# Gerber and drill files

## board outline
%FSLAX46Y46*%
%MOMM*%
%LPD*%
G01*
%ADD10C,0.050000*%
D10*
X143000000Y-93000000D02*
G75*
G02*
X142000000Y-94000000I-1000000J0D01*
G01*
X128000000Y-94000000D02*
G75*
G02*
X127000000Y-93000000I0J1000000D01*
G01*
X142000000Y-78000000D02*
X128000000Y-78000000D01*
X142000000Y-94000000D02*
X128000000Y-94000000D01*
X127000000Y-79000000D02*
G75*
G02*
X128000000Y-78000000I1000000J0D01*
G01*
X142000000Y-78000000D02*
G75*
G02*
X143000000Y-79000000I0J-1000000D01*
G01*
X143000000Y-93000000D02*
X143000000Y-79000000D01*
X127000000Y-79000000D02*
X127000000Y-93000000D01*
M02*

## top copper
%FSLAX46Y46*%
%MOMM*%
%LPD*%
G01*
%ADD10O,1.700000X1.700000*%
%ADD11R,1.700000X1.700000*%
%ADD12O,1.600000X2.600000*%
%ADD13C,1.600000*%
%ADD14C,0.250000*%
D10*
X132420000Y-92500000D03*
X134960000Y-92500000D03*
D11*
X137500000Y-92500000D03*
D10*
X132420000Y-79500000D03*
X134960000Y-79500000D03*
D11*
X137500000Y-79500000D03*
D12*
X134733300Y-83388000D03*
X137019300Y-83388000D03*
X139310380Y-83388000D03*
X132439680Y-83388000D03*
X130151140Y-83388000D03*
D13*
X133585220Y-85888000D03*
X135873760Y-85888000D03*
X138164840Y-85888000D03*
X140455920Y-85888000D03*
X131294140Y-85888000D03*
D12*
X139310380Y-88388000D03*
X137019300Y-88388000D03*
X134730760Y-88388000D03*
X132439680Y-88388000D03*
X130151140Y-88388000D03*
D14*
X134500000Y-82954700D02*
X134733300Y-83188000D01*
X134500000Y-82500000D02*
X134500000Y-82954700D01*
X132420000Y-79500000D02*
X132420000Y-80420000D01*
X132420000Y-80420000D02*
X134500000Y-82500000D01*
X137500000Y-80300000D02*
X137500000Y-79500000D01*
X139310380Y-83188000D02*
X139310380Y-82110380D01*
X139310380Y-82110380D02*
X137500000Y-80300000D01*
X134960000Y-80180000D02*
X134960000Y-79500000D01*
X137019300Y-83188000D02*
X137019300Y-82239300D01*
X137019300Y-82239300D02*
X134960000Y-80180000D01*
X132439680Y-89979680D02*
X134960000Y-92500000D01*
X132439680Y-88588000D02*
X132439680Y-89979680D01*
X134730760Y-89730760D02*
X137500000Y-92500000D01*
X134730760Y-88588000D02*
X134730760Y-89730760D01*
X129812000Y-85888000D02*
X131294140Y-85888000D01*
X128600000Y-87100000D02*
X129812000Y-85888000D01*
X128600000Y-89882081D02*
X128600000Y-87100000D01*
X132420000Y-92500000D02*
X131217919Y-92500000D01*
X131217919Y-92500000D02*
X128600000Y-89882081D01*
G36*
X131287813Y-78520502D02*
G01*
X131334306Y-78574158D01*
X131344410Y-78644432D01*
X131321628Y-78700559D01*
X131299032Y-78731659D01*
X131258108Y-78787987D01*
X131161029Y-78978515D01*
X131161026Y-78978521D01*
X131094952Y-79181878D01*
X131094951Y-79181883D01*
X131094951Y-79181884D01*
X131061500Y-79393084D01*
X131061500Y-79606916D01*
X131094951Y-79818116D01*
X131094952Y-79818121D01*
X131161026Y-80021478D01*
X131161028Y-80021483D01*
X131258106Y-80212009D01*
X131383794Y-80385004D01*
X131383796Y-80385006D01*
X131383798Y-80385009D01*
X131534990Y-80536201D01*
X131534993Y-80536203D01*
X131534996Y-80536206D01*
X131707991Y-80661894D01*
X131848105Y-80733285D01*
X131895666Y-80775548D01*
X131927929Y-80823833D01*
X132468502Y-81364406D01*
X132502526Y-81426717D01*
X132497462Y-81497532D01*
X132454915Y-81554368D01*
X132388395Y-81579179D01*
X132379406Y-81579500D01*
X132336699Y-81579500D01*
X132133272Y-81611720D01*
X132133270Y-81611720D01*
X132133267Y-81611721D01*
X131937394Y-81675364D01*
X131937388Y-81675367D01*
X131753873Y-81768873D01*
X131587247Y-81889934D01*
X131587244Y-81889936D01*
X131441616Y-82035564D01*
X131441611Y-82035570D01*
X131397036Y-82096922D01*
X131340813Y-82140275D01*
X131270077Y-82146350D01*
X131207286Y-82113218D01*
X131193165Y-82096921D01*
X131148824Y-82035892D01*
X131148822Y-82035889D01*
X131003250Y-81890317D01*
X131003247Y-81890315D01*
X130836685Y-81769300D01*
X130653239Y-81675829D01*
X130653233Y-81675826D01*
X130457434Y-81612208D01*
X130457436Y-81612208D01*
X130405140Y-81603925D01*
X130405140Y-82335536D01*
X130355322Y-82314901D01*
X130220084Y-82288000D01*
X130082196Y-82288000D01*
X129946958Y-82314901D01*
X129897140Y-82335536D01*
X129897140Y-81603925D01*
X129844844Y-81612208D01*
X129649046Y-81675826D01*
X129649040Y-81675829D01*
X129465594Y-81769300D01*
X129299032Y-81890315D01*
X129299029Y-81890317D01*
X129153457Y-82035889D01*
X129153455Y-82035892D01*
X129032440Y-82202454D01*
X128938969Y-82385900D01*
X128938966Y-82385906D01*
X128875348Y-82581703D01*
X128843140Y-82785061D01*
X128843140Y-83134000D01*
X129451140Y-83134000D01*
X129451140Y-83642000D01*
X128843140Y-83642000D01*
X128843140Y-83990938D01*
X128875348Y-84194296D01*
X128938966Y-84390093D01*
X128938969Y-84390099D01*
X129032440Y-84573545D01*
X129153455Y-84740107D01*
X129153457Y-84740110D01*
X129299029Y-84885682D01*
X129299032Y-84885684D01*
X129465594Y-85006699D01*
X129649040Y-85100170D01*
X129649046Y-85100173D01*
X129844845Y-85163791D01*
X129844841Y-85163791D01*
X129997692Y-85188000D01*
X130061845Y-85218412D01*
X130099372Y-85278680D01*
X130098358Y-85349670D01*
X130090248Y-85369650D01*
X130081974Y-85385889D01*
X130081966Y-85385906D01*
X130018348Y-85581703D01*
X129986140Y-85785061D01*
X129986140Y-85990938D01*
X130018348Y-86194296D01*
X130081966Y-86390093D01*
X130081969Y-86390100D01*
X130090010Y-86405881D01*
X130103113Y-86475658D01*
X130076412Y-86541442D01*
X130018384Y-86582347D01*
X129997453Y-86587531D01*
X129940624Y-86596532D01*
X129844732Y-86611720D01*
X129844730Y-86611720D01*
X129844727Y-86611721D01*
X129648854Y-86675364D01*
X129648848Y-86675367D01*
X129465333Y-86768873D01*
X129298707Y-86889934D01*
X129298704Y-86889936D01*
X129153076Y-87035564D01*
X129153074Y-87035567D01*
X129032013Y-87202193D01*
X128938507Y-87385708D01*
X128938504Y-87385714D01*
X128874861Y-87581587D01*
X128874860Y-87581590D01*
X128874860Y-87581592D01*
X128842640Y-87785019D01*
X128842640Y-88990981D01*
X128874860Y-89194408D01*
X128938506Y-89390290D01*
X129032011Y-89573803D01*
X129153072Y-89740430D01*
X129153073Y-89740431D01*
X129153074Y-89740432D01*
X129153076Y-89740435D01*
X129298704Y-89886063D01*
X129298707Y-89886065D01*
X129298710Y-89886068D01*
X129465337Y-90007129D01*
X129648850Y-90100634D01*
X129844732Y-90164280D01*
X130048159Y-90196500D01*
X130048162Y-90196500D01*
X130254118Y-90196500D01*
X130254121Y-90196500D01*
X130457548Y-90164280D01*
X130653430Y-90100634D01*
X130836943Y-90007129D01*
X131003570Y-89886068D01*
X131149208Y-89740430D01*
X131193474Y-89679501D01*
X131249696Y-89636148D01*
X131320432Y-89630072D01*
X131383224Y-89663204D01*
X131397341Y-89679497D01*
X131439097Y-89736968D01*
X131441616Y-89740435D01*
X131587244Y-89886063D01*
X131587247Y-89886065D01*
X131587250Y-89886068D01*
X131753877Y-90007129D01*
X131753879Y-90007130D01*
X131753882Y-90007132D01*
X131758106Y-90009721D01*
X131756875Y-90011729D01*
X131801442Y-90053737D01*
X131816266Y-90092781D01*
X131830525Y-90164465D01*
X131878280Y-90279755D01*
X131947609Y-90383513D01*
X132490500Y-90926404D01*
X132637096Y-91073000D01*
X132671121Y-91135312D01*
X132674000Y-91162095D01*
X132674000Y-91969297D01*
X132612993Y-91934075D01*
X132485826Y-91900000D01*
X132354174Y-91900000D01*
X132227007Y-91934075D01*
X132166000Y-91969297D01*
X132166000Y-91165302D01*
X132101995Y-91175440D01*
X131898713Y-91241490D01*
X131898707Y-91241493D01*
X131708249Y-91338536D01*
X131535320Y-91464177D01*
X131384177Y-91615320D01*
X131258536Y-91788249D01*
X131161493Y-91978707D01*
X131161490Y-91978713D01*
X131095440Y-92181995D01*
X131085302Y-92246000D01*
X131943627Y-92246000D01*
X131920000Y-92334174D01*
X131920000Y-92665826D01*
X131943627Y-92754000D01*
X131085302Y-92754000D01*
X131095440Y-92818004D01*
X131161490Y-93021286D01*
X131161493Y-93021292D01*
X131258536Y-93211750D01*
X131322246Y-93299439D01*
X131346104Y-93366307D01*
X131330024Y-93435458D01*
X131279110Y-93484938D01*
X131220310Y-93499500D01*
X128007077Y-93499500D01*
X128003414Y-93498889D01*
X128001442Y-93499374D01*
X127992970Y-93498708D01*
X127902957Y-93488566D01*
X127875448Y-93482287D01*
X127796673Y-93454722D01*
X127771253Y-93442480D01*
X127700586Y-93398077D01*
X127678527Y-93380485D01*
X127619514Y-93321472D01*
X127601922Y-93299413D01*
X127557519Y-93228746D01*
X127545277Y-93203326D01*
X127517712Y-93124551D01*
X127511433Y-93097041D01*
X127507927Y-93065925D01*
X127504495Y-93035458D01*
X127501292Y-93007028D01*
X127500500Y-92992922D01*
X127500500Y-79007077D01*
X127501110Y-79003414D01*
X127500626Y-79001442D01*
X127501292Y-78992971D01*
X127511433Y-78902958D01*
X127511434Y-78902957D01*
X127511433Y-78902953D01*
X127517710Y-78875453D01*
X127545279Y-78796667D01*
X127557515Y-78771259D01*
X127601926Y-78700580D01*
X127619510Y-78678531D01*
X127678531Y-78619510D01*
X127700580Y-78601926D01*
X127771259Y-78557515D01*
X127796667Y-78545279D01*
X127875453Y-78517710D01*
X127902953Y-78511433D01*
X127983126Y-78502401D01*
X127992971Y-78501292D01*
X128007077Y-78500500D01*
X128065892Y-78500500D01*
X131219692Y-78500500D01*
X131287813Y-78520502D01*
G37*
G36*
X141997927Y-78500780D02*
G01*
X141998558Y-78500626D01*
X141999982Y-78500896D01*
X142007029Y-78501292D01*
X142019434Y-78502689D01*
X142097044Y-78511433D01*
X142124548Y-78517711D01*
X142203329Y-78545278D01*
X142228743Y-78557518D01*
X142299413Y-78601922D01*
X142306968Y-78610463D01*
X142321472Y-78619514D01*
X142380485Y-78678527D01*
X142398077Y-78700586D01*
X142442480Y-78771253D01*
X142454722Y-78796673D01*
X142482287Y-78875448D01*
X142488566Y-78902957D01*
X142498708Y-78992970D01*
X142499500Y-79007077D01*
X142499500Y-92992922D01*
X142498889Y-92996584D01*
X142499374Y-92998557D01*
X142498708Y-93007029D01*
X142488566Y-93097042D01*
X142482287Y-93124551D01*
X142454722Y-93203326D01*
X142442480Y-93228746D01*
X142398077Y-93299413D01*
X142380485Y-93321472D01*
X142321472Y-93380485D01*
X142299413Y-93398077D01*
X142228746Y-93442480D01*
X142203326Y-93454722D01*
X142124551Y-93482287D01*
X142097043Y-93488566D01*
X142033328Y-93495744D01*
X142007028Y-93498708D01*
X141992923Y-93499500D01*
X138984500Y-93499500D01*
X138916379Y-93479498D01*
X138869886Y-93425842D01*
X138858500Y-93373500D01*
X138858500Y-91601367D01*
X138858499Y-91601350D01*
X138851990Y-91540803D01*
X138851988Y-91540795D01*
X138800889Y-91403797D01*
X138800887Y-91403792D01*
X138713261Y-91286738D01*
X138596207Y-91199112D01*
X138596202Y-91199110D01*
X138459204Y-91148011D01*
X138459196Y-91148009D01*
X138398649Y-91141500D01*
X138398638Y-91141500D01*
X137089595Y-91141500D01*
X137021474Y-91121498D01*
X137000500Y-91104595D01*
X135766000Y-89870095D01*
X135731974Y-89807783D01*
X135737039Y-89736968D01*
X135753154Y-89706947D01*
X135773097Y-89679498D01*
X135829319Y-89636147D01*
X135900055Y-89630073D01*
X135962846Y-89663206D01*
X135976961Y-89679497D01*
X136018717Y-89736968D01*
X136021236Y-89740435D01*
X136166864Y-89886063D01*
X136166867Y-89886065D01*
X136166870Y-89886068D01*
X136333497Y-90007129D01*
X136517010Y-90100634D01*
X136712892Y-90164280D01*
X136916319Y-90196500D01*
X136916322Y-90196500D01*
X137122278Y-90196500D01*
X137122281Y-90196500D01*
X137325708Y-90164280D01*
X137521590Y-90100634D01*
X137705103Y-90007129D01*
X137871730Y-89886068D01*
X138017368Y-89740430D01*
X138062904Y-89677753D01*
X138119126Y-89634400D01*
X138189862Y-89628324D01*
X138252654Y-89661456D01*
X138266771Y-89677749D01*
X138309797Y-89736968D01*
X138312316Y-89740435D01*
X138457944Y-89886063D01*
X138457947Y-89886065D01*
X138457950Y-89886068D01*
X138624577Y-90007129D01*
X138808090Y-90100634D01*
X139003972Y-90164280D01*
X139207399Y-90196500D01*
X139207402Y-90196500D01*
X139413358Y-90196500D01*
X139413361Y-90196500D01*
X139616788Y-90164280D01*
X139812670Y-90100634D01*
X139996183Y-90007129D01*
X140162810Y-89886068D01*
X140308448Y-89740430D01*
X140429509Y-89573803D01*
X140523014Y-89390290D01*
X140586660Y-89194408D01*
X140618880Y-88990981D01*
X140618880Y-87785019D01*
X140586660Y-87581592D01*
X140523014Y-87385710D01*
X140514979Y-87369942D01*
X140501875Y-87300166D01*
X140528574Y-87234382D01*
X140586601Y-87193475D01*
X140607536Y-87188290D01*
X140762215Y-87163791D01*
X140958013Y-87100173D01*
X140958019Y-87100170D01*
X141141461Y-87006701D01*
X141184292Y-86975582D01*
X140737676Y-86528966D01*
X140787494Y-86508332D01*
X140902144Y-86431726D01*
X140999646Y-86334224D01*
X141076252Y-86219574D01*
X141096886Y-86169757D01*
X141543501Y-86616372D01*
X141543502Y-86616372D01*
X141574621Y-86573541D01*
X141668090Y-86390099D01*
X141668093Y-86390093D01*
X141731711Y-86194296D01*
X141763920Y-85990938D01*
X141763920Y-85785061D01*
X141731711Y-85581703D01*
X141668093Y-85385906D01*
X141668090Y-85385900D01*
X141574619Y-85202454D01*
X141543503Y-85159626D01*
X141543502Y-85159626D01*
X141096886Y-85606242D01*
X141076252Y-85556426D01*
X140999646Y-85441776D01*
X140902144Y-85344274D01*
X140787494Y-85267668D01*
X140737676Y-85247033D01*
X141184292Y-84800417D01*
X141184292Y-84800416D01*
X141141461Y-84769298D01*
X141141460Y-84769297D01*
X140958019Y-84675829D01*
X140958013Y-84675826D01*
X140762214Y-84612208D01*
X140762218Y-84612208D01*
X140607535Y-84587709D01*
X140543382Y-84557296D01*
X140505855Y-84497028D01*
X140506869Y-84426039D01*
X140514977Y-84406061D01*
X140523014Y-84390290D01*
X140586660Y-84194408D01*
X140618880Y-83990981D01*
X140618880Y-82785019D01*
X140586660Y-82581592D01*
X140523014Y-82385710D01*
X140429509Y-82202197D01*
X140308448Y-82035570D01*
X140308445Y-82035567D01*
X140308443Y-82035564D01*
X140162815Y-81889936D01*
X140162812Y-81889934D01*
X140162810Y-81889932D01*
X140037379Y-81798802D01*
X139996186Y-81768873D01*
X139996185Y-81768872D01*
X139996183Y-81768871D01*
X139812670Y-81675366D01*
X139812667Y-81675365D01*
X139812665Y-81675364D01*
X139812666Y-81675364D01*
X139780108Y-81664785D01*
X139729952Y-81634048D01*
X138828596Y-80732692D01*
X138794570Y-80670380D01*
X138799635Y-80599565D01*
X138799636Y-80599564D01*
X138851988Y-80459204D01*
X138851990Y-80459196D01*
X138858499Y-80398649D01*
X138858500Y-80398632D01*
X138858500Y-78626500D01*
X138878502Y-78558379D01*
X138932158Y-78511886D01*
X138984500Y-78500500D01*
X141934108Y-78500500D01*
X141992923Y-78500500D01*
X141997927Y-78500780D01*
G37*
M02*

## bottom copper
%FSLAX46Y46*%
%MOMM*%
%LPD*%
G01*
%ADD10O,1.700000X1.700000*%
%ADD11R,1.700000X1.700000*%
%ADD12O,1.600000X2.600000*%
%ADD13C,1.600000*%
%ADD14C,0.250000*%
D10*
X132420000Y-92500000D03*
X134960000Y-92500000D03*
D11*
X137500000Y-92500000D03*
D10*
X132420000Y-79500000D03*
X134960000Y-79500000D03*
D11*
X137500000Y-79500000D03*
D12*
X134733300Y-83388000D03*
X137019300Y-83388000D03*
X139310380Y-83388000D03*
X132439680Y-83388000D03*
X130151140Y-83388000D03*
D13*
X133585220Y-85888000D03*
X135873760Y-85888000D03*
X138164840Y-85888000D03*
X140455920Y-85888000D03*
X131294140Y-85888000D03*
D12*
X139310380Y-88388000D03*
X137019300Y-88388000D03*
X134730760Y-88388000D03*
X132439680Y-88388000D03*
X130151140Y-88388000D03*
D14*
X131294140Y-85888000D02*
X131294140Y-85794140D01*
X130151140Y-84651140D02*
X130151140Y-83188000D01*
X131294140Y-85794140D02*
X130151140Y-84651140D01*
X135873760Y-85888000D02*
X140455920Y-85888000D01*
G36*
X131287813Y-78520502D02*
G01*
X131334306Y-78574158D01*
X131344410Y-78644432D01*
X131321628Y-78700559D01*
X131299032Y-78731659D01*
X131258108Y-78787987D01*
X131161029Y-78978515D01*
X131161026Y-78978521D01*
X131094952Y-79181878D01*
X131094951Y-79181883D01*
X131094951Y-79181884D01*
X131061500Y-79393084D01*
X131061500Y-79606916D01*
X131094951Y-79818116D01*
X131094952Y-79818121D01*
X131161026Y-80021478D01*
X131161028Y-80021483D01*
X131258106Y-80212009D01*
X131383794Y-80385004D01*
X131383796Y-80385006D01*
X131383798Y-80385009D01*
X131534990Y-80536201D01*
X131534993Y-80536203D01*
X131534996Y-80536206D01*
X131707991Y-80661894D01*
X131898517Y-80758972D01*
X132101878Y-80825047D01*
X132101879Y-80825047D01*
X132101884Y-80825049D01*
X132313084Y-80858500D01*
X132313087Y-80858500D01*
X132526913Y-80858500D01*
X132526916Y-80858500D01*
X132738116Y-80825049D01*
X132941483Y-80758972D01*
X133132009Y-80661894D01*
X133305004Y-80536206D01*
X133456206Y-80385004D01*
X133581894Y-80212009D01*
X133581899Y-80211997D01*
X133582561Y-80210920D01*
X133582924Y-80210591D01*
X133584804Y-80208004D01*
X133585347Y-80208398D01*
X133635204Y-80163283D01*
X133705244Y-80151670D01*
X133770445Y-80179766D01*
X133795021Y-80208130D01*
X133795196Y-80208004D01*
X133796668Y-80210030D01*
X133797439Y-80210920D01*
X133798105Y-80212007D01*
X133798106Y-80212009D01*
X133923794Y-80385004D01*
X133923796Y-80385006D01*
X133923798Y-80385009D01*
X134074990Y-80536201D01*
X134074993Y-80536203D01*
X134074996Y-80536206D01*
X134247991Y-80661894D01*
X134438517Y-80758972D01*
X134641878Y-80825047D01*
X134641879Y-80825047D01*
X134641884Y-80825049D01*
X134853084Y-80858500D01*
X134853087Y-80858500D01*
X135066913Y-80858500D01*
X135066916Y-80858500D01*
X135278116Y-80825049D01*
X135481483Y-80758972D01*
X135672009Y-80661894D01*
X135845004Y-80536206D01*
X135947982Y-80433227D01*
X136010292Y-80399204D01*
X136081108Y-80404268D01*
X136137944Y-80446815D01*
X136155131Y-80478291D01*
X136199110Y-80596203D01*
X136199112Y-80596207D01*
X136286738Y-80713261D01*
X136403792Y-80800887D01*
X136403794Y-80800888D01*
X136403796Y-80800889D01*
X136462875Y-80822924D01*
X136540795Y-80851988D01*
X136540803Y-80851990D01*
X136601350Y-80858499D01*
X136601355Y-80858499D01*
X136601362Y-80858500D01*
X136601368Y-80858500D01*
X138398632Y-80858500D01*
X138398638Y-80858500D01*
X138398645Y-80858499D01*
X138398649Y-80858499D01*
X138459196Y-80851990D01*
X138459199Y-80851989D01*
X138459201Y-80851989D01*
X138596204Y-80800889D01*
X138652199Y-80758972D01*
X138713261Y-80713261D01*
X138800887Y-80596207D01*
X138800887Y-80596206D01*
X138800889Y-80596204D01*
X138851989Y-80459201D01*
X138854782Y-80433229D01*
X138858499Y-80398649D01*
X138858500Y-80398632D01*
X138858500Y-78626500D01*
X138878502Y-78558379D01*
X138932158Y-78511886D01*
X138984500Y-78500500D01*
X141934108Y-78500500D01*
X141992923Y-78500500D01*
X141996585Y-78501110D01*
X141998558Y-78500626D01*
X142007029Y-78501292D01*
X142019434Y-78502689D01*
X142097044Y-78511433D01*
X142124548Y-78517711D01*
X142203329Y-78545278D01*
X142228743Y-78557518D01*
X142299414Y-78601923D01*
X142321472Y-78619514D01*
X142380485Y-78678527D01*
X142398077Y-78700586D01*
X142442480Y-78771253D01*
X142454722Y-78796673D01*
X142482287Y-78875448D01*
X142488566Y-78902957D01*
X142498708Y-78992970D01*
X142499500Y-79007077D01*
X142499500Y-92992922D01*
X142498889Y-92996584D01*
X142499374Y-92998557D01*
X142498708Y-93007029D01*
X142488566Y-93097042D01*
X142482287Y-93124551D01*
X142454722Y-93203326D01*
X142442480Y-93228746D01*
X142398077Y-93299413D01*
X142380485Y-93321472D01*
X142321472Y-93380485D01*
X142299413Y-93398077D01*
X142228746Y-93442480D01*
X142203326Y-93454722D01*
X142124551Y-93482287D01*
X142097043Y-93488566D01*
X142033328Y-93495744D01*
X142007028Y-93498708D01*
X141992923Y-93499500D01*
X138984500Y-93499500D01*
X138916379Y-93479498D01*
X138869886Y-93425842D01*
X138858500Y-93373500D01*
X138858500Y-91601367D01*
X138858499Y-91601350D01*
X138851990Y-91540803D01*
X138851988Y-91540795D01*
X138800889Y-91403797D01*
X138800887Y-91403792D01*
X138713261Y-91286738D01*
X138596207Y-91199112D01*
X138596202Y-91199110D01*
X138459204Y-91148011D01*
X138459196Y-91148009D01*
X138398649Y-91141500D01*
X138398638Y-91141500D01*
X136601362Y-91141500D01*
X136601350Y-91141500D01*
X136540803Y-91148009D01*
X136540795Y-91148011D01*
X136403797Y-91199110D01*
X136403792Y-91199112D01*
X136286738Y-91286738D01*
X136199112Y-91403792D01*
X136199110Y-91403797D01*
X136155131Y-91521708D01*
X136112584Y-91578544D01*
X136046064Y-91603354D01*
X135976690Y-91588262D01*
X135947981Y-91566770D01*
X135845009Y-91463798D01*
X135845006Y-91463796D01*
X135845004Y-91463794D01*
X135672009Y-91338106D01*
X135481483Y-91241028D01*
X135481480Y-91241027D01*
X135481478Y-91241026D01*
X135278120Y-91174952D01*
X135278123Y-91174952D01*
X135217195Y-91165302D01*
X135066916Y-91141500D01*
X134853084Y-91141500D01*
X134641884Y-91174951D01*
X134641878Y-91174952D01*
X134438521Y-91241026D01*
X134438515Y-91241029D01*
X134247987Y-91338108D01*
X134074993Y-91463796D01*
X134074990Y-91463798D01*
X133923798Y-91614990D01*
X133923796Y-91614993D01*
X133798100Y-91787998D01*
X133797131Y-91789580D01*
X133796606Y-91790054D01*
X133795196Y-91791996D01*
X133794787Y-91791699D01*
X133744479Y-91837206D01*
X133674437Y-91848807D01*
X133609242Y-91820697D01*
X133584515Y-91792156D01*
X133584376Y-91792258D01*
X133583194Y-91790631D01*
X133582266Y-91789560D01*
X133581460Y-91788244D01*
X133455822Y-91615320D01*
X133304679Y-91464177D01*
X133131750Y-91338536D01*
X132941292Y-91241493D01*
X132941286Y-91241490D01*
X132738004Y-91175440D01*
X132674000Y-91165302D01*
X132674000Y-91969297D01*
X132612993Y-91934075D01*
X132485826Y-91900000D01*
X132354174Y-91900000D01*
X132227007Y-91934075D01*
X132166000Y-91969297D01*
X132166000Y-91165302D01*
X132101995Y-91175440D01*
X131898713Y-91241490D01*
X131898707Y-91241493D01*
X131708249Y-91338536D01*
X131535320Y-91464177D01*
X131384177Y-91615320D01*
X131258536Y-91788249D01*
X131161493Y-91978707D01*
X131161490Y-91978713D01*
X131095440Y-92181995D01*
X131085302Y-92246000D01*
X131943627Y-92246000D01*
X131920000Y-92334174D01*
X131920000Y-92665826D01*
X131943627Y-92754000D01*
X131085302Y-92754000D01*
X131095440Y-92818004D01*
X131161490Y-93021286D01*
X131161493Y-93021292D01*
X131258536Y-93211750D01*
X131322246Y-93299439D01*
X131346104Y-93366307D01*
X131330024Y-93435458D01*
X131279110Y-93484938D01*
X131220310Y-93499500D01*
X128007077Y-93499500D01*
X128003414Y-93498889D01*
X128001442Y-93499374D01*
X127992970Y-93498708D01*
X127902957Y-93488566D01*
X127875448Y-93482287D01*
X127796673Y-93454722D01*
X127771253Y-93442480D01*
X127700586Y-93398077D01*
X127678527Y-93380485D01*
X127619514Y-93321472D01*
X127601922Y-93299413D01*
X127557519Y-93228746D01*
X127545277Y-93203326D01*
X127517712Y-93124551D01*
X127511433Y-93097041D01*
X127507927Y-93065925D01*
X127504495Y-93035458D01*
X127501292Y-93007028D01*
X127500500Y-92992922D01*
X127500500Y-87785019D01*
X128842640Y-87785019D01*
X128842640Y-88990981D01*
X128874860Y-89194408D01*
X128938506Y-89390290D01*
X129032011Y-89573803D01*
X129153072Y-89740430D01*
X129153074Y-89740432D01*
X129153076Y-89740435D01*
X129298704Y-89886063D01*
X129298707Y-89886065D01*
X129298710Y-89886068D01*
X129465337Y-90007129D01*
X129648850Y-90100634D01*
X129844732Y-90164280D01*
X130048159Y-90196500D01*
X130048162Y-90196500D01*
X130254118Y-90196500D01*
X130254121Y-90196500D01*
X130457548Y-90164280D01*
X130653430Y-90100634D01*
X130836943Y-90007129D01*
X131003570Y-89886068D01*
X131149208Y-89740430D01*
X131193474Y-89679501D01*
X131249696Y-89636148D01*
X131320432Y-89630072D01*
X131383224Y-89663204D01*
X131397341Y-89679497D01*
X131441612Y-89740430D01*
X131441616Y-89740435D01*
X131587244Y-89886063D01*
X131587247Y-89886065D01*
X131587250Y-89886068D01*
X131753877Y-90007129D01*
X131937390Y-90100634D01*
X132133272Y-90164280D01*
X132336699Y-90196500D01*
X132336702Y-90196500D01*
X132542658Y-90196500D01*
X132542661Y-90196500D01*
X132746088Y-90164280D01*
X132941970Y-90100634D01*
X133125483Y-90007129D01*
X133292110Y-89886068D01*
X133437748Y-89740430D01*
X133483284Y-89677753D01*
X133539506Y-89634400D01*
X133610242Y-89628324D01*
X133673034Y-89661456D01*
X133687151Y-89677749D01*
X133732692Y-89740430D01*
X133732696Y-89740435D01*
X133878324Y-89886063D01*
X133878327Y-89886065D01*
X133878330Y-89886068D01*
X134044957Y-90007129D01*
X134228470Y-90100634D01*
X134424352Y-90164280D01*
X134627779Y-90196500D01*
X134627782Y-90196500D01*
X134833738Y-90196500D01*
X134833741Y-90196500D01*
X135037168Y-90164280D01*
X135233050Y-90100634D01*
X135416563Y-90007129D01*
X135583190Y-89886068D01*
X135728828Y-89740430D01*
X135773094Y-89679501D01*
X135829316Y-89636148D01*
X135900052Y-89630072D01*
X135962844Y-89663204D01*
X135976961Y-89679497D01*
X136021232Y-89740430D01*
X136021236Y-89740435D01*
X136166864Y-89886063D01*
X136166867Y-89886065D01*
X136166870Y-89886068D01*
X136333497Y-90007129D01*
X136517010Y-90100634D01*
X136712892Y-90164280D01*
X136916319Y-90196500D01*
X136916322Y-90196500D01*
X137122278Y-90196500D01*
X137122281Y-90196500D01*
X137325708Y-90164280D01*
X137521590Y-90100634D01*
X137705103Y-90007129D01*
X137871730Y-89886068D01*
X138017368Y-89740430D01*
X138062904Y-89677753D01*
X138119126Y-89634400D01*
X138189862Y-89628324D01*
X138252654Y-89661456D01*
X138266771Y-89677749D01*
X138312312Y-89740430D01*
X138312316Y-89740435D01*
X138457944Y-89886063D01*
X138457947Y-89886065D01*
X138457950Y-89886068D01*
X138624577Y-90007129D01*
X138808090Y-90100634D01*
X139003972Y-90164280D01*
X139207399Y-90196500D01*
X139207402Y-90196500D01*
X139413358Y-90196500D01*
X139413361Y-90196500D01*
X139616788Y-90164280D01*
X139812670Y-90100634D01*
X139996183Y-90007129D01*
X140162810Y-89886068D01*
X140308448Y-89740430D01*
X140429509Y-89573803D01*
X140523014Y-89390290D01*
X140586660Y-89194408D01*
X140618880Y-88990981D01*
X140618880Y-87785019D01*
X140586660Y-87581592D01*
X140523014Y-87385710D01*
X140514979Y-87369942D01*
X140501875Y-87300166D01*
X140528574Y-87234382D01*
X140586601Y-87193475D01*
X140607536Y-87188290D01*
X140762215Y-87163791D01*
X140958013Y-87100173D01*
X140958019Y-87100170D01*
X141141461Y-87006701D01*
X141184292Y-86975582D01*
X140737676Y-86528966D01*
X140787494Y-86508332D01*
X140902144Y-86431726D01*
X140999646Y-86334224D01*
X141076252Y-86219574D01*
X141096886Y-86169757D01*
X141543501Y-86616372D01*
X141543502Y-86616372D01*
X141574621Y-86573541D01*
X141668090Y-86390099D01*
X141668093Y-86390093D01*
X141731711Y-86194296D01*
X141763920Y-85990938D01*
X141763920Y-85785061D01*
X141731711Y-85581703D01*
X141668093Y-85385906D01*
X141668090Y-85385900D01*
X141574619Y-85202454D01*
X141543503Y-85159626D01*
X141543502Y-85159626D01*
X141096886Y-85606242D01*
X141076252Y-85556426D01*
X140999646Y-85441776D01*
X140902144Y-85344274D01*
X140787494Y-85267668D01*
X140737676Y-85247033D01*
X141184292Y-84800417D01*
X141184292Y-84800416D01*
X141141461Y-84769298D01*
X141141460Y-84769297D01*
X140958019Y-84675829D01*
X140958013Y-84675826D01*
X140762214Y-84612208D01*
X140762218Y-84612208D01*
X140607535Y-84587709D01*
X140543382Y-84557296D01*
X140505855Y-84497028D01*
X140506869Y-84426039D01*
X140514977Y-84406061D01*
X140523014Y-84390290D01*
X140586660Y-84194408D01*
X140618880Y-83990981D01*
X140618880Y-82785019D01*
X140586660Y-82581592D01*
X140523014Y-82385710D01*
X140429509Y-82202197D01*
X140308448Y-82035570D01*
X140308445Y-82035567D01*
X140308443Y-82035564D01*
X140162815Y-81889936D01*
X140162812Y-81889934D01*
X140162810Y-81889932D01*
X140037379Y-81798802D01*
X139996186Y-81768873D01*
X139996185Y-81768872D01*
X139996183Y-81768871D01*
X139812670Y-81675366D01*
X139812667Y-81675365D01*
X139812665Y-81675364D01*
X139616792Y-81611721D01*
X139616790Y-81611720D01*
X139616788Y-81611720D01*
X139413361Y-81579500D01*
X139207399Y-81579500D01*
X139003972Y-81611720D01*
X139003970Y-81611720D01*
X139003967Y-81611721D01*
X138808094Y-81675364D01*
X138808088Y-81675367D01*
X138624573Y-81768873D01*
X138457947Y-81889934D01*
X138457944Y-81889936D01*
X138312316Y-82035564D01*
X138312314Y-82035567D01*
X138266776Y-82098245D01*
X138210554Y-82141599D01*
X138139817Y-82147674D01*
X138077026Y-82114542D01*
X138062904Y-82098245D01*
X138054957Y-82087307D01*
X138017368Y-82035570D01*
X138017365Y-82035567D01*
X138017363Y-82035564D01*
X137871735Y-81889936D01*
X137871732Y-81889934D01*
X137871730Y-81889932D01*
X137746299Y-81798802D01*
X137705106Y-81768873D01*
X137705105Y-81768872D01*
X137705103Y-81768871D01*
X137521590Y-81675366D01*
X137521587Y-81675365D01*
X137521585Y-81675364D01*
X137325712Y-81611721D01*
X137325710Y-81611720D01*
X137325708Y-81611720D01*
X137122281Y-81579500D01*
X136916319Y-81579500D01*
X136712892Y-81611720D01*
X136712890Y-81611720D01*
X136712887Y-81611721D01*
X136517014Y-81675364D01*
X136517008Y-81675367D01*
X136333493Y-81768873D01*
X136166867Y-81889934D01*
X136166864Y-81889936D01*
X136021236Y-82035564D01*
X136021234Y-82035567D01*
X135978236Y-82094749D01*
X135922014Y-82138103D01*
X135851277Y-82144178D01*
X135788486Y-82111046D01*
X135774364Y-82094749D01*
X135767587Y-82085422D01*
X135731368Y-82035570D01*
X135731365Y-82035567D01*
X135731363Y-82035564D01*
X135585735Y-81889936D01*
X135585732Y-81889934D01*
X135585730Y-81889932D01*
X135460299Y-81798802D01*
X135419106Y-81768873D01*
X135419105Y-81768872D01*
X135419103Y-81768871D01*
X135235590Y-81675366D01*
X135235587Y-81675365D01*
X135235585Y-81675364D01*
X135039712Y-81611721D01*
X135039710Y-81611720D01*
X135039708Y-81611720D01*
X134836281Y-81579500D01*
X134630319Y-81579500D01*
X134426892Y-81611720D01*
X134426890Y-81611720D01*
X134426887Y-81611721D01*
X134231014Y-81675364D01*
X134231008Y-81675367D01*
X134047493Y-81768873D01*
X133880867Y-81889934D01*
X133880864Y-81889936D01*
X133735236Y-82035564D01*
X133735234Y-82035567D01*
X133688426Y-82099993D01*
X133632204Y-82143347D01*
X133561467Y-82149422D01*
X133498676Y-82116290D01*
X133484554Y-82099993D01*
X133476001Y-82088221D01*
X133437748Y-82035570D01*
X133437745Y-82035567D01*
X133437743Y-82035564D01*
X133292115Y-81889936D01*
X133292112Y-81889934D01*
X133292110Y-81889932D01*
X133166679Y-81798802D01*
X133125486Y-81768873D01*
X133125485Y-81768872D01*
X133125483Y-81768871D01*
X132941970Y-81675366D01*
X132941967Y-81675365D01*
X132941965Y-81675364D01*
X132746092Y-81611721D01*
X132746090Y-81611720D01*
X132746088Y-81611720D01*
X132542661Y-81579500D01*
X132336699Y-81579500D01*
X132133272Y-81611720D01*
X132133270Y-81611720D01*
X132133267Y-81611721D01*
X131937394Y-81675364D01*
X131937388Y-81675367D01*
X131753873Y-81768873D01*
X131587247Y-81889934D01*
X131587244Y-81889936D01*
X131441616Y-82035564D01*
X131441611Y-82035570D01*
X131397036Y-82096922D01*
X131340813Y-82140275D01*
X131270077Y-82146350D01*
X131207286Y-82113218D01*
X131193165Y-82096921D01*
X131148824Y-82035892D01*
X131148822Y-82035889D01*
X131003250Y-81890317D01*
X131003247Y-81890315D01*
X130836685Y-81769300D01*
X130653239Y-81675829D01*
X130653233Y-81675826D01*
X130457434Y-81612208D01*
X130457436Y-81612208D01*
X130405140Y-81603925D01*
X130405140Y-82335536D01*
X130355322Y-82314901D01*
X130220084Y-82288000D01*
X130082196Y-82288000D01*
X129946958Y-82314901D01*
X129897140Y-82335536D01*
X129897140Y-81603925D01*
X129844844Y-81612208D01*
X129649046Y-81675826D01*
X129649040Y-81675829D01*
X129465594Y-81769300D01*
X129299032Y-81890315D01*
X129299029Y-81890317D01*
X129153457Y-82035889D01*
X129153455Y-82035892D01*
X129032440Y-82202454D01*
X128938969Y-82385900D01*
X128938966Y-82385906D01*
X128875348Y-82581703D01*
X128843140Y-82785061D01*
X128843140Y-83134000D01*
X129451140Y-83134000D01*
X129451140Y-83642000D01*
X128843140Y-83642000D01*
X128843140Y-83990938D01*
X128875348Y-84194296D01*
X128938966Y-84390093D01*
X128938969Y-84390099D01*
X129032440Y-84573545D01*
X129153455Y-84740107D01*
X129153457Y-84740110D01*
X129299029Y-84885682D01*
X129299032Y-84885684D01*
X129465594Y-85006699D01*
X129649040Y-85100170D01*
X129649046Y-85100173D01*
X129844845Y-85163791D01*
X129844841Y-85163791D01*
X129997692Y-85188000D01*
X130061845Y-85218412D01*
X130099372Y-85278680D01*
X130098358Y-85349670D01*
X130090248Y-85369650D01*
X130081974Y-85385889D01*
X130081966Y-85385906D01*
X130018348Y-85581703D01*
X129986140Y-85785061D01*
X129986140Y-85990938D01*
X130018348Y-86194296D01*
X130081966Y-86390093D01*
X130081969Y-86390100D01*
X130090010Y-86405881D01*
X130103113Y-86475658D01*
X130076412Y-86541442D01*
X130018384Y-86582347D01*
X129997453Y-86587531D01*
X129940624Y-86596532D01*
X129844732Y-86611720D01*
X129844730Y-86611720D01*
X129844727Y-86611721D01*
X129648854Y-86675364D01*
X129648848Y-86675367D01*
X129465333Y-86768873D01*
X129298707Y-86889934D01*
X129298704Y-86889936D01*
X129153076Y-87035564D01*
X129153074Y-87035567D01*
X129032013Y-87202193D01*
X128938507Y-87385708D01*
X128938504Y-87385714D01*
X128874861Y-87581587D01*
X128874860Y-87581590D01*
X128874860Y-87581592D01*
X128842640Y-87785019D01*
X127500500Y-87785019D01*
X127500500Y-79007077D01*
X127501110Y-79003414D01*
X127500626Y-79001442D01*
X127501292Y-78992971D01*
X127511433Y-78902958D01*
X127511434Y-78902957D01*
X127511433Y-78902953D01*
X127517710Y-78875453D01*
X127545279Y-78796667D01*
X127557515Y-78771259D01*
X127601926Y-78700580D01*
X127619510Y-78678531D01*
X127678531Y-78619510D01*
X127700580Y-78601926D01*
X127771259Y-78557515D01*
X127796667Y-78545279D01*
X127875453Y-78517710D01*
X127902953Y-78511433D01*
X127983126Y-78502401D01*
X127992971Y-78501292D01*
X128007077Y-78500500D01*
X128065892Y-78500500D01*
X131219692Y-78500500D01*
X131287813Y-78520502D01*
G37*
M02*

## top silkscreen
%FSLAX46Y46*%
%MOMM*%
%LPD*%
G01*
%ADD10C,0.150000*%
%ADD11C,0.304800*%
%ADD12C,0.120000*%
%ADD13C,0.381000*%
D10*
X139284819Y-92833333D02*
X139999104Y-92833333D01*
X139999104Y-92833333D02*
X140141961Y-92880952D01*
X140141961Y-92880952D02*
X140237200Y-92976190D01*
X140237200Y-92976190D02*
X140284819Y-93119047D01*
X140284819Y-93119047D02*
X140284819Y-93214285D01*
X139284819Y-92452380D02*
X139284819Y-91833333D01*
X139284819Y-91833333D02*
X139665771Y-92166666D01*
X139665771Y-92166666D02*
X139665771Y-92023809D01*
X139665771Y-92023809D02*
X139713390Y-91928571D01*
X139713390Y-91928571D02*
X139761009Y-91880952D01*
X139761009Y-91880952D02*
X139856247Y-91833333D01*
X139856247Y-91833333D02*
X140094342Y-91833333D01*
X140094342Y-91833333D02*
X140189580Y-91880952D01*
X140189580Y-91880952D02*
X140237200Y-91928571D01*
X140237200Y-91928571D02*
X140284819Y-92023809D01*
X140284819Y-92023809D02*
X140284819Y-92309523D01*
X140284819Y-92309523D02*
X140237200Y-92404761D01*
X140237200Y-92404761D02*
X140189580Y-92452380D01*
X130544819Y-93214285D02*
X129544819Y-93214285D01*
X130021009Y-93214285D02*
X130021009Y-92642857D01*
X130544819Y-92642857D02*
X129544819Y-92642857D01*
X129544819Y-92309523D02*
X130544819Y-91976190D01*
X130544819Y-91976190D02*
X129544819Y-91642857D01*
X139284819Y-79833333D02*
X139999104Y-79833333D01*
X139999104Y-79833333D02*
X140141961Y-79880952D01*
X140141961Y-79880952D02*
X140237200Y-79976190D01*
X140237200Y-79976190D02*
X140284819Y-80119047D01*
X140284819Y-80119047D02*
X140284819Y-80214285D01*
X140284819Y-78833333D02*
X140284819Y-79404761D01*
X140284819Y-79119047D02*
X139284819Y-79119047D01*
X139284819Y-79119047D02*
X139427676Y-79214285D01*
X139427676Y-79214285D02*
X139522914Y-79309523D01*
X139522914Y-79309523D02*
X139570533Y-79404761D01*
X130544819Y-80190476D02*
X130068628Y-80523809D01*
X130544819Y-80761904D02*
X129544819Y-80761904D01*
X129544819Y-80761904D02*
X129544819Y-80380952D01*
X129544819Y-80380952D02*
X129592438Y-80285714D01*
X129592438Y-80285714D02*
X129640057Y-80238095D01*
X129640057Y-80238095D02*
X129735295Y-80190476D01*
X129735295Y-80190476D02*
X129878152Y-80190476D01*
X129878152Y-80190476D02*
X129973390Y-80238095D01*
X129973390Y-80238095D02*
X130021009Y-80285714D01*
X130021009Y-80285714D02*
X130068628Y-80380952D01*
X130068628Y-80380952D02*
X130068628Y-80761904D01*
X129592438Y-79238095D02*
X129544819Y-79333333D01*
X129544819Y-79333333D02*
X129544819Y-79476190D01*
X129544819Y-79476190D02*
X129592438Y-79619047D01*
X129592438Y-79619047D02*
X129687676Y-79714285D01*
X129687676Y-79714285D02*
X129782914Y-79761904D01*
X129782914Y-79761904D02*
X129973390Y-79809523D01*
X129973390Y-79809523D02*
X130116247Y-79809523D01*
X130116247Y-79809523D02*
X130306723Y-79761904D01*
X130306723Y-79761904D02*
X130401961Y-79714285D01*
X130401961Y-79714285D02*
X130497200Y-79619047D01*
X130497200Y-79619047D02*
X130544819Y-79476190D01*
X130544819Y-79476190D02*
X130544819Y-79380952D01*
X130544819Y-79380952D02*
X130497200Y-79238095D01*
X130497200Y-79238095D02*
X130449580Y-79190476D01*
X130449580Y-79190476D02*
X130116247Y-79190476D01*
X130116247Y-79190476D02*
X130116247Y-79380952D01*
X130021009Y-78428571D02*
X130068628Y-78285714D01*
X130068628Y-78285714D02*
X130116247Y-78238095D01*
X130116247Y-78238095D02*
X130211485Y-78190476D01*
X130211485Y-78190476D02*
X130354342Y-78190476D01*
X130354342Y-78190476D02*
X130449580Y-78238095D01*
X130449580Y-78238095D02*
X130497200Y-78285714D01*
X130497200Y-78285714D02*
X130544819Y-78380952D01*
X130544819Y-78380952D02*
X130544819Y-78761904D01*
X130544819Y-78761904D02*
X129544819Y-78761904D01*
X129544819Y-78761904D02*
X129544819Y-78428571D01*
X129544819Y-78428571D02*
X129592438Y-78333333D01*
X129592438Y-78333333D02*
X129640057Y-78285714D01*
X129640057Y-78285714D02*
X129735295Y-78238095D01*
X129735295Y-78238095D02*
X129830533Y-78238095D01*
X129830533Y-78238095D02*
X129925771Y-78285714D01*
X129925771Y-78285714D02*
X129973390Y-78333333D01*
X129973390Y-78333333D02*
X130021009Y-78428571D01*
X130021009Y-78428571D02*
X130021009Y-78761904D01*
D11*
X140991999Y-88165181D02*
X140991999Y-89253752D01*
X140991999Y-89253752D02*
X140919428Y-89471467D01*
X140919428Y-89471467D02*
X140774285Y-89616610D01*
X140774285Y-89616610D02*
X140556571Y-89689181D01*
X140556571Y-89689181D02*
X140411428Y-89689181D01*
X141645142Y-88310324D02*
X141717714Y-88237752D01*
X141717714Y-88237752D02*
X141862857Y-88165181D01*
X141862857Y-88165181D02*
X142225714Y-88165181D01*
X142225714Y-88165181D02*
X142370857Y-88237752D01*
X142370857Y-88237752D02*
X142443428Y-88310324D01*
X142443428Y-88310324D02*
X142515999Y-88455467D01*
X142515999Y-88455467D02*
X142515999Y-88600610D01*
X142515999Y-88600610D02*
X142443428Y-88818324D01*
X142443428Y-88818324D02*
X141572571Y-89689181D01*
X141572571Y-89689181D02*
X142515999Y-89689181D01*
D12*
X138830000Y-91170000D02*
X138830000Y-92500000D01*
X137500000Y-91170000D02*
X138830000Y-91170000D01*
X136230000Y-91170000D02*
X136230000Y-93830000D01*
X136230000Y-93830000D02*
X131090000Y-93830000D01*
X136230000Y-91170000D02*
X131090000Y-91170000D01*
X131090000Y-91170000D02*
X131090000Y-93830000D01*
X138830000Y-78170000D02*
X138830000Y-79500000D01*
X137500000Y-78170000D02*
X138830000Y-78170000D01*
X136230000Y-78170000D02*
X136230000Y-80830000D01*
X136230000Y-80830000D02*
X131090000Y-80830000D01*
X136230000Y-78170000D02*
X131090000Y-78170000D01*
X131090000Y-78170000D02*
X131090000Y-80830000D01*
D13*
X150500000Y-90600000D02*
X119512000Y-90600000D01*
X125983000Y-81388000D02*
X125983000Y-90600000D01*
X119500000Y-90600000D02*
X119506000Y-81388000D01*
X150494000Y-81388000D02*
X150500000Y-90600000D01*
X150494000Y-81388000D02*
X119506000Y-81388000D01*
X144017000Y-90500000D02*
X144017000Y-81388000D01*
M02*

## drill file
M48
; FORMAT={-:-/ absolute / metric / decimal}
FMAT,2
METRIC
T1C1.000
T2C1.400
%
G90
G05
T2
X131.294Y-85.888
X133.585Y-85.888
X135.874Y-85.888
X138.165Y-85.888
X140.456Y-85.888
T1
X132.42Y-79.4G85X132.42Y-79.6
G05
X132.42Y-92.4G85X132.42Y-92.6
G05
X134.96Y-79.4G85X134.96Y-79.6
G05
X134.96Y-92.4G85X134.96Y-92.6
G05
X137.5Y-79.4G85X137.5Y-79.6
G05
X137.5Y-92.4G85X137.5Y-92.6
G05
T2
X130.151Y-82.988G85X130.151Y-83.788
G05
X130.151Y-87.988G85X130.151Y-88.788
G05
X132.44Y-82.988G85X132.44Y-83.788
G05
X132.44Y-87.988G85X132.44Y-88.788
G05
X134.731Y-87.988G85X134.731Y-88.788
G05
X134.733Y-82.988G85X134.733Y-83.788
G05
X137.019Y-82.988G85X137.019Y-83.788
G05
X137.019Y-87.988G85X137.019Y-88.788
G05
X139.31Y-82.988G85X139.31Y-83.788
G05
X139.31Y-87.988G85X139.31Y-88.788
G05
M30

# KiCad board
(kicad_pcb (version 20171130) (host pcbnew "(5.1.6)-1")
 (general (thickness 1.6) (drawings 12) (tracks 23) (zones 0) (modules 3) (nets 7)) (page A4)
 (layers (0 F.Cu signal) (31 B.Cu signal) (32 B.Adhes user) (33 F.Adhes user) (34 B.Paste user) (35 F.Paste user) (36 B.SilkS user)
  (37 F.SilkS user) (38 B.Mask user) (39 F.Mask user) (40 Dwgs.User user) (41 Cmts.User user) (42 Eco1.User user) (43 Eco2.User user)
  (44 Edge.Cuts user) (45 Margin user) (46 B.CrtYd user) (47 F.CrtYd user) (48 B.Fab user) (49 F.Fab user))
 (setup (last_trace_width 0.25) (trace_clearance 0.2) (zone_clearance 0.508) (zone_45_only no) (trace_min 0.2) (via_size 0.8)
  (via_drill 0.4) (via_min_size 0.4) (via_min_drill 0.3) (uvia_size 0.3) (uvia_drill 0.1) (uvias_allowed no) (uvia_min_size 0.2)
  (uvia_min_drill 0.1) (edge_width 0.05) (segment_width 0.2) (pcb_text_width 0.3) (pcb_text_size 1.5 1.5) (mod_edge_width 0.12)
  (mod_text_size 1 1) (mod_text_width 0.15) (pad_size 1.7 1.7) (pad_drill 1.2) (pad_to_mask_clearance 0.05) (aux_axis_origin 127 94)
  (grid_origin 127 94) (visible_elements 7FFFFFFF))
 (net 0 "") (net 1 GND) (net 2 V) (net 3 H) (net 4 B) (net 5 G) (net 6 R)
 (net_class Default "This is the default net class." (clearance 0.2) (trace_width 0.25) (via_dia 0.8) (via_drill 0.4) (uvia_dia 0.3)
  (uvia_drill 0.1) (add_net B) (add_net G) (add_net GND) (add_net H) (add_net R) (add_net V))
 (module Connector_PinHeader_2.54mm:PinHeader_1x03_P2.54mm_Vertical (layer F.Cu) (at 137.5 92.5 270)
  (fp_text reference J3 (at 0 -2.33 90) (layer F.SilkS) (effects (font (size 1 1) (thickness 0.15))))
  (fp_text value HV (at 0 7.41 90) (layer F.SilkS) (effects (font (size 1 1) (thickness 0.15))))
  (fp_line (start -1.33 -1.33) (end 0 -1.33) (layer F.SilkS) (width 0.12))
  (fp_line (start -1.33 0) (end -1.33 -1.33) (layer F.SilkS) (width 0.12))
  (fp_line (start -1.33 1.27) (end 1.33 1.27) (layer F.SilkS) (width 0.12))
  (fp_line (start 1.33 1.27) (end 1.33 6.41) (layer F.SilkS) (width 0.12))
  (fp_line (start -1.33 1.27) (end -1.33 6.41) (layer F.SilkS) (width 0.12))
  (fp_line (start -1.33 6.41) (end 1.33 6.41) (layer F.SilkS) (width 0.12))
  (pad 3 thru_hole oval (at 0 5.08 270) (size 1.7 1.7) (drill oval 1.2 1) (layers *.Cu *.Mask) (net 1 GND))
  (pad 2 thru_hole oval (at 0 2.54 270) (size 1.7 1.7) (drill oval 1.2 1) (layers *.Cu *.Mask) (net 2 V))
  (pad 1 thru_hole rect (at 0 0 270) (size 1.7 1.7) (drill oval 1.2 1) (layers *.Cu *.Mask) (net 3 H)))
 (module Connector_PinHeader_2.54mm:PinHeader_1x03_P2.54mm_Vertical (layer F.Cu) (at 137.5 79.5 270)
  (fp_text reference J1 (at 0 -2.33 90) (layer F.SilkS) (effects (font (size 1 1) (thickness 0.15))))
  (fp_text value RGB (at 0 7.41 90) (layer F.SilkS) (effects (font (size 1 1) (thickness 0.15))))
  (fp_line (start -1.33 -1.33) (end 0 -1.33) (layer F.SilkS) (width 0.12))
  (fp_line (start -1.33 0) (end -1.33 -1.33) (layer F.SilkS) (width 0.12))
  (fp_line (start -1.33 1.27) (end 1.33 1.27) (layer F.SilkS) (width 0.12))
  (fp_line (start 1.33 1.27) (end 1.33 6.41) (layer F.SilkS) (width 0.12))
  (fp_line (start -1.33 1.27) (end -1.33 6.41) (layer F.SilkS) (width 0.12))
  (fp_line (start -1.33 6.41) (end 1.33 6.41) (layer F.SilkS) (width 0.12))
  (pad 3 thru_hole oval (at 0 5.08 270) (size 1.7 1.7) (drill oval 1.2 1) (layers *.Cu *.Mask) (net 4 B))
  (pad 2 thru_hole oval (at 0 2.54 270) (size 1.7 1.7) (drill oval 1.2 1) (layers *.Cu *.Mask) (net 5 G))
  (pad 1 thru_hole rect (at 0 0 270) (size 1.7 1.7) (drill oval 1.2 1) (layers *.Cu *.Mask) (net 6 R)))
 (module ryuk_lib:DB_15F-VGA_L (layer F.Cu) (at 135 96.5)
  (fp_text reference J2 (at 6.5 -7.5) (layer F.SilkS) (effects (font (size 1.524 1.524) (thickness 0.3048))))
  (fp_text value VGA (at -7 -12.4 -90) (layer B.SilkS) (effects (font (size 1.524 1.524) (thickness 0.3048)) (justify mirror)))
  (fp_line (start 15.5 -5.9) (end -15.488 -5.9) (layer F.SilkS) (width 0.381))
  (fp_line (start -9.017 -15.112) (end -9.017 -5.9) (layer F.SilkS) (width 0.381))
  (fp_line (start -15.5 -5.9) (end -15.494 -15.112) (layer F.SilkS) (width 0.381))
  (fp_line (start 15.494 -15.112) (end 15.5 -5.9) (layer F.SilkS) (width 0.381))
  (fp_line (start 15.494 -15.112) (end -15.494 -15.112) (layer F.SilkS) (width 0.381))
  (fp_line (start 9.017 -6) (end 9.017 -15.112) (layer F.SilkS) (width 0.381))
  (pad 3 thru_hole oval (at -0.2667 -13.112) (size 1.6 2.6) (drill oval 1.4 2.2) (layers *.Cu *.Mask) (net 4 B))
  (pad 2 thru_hole oval (at 2.0193 -13.112) (size 1.6 2.6) (drill oval 1.4 2.2) (layers *.Cu *.Mask) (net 5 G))
  (pad 1 thru_hole oval (at 4.31038 -13.112) (size 1.6 2.6) (drill oval 1.4 2.2) (layers *.Cu *.Mask) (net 6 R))
  (pad 4 thru_hole oval (at -2.56032 -13.112) (size 1.6 2.6) (drill oval 1.4 2.2) (layers *.Cu *.Mask))
  (pad 5 thru_hole oval (at -4.84886 -13.112) (size 1.6 2.6) (drill oval 1.4 2.2) (layers *.Cu *.Mask) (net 1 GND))
  (pad 9 thru_hole circle (at -1.41478 -10.612) (size 1.6 1.6) (drill 1.4) (layers *.Cu *.Mask))
  (pad 8 thru_hole circle (at 0.87376 -10.612) (size 1.6 1.6) (drill 1.4) (layers *.Cu *.Mask) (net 1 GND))
  (pad 7 thru_hole circle (at 3.16484 -10.612) (size 1.6 1.6) (drill 1.4) (layers *.Cu *.Mask) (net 1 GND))
  (pad 6 thru_hole circle (at 5.45592 -10.612) (size 1.6 1.6) (drill 1.4) (layers *.Cu *.Mask) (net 1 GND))
  (pad 10 thru_hole circle (at -3.70586 -10.612) (size 1.6 1.6) (drill 1.4) (layers *.Cu *.Mask) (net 1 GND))
  (pad 11 thru_hole oval (at 4.31038 -8.112) (size 1.6 2.6) (drill oval 1.4 2.2) (layers *.Cu *.Mask))
  (pad 12 thru_hole oval (at 2.0193 -8.112) (size 1.6 2.6) (drill oval 1.4 2.2) (layers *.Cu *.Mask))
  (pad 13 thru_hole oval (at -0.26924 -8.112) (size 1.6 2.6) (drill oval 1.4 2.2) (layers *.Cu *.Mask) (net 3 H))
  (pad 14 thru_hole oval (at -2.56032 -8.112) (size 1.6 2.6) (drill oval 1.4 2.2) (layers *.Cu *.Mask) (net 2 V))
  (pad 15 thru_hole oval (at -4.84886 -8.112) (size 1.6 2.6) (drill oval 1.4 2.2) (layers *.Cu *.Mask)))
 (gr_arc (start 142 93) (end 142 94) (angle -90) (layer Edge.Cuts) (width 0.05))
 (gr_arc (start 128 93) (end 127 93) (angle -90) (layer Edge.Cuts) (width 0.05))
 (gr_line (start 142 78) (end 128 78) (layer Edge.Cuts) (width 0.05))
 (gr_line (start 142 94) (end 128 94) (layer Edge.Cuts) (width 0.05))
 (gr_arc (start 128 79) (end 128 78) (angle -90) (layer Edge.Cuts) (width 0.05))
 (gr_arc (start 142 79) (end 143 79) (angle -90) (layer Edge.Cuts) (width 0.05))
 (gr_line (start 143 93) (end 143 79) (layer Edge.Cuts) (width 0.05))
 (gr_line (start 127 79) (end 127 93) (layer Edge.Cuts) (width 0.05))
 (segment (start 134.5 82.9547) (end 134.7333 83.188) (width 0.25) (layer F.Cu) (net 4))
 (segment (start 134.5 82.5) (end 134.5 82.9547) (width 0.25) (layer F.Cu) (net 4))
 (segment (start 132.42 79.5) (end 132.42 80.42) (width 0.25) (layer F.Cu) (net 4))
 (segment (start 132.42 80.42) (end 134.5 82.5) (width 0.25) (layer F.Cu) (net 4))
 (segment (start 137.5 80.3) (end 137.5 79.5) (width 0.25) (layer F.Cu) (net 6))
 (segment (start 139.31038 83.188) (end 139.31038 82.11038) (width 0.25) (layer F.Cu) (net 6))
 (segment (start 139.31038 82.11038) (end 137.5 80.3) (width 0.25) (layer F.Cu) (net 6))
 (segment (start 134.96 80.18) (end 134.96 79.5) (width 0.25) (layer F.Cu) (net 5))
 (segment (start 137.0193 83.188) (end 137.0193 82.2393) (width 0.25) (layer F.Cu) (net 5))
 (segment (start 137.0193 82.2393) (end 134.96 80.18) (width 0.25) (layer F.Cu) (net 5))
 (segment (start 132.43968 89.97968) (end 134.96 92.5) (width 0.25) (layer F.Cu) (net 2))
 (segment (start 132.43968 88.588) (end 132.43968 89.97968) (width 0.25) (layer F.Cu) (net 2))
 (segment (start 134.73076 89.73076) (end 137.5 92.5) (width 0.25) (layer F.Cu) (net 3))
 (segment (start 134.73076 88.588) (end 134.73076 89.73076) (width 0.25) (layer F.Cu) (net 3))
 (segment (start 131.29414 85.888) (end 131.29414 85.79414) (width 0.25) (layer B.Cu) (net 1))
 (segment (start 130.15114 84.65114) (end 130.15114 83.188) (width 0.25) (layer B.Cu) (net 1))
 (segment (start 131.29414 85.79414) (end 130.15114 84.65114) (width 0.25) (layer B.Cu) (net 1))
 (segment (start 135.87376 85.888) (end 140.45592 85.888) (width 0.25) (layer B.Cu) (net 1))
 (segment (start 129.812 85.888) (end 131.29414 85.888) (width 0.25) (layer F.Cu) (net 1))
 (segment (start 128.6 87.1) (end 129.812 85.888) (width 0.25) (layer F.Cu) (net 1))
 (segment (start 128.6 89.882081) (end 128.6 87.1) (width 0.25) (layer F.Cu) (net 1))
 (segment (start 132.42 92.5) (end 131.217919 92.5) (width 0.25) (layer F.Cu) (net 1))
 (segment (start 131.217919 92.5) (end 128.6 89.882081) (width 0.25) (layer F.Cu) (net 1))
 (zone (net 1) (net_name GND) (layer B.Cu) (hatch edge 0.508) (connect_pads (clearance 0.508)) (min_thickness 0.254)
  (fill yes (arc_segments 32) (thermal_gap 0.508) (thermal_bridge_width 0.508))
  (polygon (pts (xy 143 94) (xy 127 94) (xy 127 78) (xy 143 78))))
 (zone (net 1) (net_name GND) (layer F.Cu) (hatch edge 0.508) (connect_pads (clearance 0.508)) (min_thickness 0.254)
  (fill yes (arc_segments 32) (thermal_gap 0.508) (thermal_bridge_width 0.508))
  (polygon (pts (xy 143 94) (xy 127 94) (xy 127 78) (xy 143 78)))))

